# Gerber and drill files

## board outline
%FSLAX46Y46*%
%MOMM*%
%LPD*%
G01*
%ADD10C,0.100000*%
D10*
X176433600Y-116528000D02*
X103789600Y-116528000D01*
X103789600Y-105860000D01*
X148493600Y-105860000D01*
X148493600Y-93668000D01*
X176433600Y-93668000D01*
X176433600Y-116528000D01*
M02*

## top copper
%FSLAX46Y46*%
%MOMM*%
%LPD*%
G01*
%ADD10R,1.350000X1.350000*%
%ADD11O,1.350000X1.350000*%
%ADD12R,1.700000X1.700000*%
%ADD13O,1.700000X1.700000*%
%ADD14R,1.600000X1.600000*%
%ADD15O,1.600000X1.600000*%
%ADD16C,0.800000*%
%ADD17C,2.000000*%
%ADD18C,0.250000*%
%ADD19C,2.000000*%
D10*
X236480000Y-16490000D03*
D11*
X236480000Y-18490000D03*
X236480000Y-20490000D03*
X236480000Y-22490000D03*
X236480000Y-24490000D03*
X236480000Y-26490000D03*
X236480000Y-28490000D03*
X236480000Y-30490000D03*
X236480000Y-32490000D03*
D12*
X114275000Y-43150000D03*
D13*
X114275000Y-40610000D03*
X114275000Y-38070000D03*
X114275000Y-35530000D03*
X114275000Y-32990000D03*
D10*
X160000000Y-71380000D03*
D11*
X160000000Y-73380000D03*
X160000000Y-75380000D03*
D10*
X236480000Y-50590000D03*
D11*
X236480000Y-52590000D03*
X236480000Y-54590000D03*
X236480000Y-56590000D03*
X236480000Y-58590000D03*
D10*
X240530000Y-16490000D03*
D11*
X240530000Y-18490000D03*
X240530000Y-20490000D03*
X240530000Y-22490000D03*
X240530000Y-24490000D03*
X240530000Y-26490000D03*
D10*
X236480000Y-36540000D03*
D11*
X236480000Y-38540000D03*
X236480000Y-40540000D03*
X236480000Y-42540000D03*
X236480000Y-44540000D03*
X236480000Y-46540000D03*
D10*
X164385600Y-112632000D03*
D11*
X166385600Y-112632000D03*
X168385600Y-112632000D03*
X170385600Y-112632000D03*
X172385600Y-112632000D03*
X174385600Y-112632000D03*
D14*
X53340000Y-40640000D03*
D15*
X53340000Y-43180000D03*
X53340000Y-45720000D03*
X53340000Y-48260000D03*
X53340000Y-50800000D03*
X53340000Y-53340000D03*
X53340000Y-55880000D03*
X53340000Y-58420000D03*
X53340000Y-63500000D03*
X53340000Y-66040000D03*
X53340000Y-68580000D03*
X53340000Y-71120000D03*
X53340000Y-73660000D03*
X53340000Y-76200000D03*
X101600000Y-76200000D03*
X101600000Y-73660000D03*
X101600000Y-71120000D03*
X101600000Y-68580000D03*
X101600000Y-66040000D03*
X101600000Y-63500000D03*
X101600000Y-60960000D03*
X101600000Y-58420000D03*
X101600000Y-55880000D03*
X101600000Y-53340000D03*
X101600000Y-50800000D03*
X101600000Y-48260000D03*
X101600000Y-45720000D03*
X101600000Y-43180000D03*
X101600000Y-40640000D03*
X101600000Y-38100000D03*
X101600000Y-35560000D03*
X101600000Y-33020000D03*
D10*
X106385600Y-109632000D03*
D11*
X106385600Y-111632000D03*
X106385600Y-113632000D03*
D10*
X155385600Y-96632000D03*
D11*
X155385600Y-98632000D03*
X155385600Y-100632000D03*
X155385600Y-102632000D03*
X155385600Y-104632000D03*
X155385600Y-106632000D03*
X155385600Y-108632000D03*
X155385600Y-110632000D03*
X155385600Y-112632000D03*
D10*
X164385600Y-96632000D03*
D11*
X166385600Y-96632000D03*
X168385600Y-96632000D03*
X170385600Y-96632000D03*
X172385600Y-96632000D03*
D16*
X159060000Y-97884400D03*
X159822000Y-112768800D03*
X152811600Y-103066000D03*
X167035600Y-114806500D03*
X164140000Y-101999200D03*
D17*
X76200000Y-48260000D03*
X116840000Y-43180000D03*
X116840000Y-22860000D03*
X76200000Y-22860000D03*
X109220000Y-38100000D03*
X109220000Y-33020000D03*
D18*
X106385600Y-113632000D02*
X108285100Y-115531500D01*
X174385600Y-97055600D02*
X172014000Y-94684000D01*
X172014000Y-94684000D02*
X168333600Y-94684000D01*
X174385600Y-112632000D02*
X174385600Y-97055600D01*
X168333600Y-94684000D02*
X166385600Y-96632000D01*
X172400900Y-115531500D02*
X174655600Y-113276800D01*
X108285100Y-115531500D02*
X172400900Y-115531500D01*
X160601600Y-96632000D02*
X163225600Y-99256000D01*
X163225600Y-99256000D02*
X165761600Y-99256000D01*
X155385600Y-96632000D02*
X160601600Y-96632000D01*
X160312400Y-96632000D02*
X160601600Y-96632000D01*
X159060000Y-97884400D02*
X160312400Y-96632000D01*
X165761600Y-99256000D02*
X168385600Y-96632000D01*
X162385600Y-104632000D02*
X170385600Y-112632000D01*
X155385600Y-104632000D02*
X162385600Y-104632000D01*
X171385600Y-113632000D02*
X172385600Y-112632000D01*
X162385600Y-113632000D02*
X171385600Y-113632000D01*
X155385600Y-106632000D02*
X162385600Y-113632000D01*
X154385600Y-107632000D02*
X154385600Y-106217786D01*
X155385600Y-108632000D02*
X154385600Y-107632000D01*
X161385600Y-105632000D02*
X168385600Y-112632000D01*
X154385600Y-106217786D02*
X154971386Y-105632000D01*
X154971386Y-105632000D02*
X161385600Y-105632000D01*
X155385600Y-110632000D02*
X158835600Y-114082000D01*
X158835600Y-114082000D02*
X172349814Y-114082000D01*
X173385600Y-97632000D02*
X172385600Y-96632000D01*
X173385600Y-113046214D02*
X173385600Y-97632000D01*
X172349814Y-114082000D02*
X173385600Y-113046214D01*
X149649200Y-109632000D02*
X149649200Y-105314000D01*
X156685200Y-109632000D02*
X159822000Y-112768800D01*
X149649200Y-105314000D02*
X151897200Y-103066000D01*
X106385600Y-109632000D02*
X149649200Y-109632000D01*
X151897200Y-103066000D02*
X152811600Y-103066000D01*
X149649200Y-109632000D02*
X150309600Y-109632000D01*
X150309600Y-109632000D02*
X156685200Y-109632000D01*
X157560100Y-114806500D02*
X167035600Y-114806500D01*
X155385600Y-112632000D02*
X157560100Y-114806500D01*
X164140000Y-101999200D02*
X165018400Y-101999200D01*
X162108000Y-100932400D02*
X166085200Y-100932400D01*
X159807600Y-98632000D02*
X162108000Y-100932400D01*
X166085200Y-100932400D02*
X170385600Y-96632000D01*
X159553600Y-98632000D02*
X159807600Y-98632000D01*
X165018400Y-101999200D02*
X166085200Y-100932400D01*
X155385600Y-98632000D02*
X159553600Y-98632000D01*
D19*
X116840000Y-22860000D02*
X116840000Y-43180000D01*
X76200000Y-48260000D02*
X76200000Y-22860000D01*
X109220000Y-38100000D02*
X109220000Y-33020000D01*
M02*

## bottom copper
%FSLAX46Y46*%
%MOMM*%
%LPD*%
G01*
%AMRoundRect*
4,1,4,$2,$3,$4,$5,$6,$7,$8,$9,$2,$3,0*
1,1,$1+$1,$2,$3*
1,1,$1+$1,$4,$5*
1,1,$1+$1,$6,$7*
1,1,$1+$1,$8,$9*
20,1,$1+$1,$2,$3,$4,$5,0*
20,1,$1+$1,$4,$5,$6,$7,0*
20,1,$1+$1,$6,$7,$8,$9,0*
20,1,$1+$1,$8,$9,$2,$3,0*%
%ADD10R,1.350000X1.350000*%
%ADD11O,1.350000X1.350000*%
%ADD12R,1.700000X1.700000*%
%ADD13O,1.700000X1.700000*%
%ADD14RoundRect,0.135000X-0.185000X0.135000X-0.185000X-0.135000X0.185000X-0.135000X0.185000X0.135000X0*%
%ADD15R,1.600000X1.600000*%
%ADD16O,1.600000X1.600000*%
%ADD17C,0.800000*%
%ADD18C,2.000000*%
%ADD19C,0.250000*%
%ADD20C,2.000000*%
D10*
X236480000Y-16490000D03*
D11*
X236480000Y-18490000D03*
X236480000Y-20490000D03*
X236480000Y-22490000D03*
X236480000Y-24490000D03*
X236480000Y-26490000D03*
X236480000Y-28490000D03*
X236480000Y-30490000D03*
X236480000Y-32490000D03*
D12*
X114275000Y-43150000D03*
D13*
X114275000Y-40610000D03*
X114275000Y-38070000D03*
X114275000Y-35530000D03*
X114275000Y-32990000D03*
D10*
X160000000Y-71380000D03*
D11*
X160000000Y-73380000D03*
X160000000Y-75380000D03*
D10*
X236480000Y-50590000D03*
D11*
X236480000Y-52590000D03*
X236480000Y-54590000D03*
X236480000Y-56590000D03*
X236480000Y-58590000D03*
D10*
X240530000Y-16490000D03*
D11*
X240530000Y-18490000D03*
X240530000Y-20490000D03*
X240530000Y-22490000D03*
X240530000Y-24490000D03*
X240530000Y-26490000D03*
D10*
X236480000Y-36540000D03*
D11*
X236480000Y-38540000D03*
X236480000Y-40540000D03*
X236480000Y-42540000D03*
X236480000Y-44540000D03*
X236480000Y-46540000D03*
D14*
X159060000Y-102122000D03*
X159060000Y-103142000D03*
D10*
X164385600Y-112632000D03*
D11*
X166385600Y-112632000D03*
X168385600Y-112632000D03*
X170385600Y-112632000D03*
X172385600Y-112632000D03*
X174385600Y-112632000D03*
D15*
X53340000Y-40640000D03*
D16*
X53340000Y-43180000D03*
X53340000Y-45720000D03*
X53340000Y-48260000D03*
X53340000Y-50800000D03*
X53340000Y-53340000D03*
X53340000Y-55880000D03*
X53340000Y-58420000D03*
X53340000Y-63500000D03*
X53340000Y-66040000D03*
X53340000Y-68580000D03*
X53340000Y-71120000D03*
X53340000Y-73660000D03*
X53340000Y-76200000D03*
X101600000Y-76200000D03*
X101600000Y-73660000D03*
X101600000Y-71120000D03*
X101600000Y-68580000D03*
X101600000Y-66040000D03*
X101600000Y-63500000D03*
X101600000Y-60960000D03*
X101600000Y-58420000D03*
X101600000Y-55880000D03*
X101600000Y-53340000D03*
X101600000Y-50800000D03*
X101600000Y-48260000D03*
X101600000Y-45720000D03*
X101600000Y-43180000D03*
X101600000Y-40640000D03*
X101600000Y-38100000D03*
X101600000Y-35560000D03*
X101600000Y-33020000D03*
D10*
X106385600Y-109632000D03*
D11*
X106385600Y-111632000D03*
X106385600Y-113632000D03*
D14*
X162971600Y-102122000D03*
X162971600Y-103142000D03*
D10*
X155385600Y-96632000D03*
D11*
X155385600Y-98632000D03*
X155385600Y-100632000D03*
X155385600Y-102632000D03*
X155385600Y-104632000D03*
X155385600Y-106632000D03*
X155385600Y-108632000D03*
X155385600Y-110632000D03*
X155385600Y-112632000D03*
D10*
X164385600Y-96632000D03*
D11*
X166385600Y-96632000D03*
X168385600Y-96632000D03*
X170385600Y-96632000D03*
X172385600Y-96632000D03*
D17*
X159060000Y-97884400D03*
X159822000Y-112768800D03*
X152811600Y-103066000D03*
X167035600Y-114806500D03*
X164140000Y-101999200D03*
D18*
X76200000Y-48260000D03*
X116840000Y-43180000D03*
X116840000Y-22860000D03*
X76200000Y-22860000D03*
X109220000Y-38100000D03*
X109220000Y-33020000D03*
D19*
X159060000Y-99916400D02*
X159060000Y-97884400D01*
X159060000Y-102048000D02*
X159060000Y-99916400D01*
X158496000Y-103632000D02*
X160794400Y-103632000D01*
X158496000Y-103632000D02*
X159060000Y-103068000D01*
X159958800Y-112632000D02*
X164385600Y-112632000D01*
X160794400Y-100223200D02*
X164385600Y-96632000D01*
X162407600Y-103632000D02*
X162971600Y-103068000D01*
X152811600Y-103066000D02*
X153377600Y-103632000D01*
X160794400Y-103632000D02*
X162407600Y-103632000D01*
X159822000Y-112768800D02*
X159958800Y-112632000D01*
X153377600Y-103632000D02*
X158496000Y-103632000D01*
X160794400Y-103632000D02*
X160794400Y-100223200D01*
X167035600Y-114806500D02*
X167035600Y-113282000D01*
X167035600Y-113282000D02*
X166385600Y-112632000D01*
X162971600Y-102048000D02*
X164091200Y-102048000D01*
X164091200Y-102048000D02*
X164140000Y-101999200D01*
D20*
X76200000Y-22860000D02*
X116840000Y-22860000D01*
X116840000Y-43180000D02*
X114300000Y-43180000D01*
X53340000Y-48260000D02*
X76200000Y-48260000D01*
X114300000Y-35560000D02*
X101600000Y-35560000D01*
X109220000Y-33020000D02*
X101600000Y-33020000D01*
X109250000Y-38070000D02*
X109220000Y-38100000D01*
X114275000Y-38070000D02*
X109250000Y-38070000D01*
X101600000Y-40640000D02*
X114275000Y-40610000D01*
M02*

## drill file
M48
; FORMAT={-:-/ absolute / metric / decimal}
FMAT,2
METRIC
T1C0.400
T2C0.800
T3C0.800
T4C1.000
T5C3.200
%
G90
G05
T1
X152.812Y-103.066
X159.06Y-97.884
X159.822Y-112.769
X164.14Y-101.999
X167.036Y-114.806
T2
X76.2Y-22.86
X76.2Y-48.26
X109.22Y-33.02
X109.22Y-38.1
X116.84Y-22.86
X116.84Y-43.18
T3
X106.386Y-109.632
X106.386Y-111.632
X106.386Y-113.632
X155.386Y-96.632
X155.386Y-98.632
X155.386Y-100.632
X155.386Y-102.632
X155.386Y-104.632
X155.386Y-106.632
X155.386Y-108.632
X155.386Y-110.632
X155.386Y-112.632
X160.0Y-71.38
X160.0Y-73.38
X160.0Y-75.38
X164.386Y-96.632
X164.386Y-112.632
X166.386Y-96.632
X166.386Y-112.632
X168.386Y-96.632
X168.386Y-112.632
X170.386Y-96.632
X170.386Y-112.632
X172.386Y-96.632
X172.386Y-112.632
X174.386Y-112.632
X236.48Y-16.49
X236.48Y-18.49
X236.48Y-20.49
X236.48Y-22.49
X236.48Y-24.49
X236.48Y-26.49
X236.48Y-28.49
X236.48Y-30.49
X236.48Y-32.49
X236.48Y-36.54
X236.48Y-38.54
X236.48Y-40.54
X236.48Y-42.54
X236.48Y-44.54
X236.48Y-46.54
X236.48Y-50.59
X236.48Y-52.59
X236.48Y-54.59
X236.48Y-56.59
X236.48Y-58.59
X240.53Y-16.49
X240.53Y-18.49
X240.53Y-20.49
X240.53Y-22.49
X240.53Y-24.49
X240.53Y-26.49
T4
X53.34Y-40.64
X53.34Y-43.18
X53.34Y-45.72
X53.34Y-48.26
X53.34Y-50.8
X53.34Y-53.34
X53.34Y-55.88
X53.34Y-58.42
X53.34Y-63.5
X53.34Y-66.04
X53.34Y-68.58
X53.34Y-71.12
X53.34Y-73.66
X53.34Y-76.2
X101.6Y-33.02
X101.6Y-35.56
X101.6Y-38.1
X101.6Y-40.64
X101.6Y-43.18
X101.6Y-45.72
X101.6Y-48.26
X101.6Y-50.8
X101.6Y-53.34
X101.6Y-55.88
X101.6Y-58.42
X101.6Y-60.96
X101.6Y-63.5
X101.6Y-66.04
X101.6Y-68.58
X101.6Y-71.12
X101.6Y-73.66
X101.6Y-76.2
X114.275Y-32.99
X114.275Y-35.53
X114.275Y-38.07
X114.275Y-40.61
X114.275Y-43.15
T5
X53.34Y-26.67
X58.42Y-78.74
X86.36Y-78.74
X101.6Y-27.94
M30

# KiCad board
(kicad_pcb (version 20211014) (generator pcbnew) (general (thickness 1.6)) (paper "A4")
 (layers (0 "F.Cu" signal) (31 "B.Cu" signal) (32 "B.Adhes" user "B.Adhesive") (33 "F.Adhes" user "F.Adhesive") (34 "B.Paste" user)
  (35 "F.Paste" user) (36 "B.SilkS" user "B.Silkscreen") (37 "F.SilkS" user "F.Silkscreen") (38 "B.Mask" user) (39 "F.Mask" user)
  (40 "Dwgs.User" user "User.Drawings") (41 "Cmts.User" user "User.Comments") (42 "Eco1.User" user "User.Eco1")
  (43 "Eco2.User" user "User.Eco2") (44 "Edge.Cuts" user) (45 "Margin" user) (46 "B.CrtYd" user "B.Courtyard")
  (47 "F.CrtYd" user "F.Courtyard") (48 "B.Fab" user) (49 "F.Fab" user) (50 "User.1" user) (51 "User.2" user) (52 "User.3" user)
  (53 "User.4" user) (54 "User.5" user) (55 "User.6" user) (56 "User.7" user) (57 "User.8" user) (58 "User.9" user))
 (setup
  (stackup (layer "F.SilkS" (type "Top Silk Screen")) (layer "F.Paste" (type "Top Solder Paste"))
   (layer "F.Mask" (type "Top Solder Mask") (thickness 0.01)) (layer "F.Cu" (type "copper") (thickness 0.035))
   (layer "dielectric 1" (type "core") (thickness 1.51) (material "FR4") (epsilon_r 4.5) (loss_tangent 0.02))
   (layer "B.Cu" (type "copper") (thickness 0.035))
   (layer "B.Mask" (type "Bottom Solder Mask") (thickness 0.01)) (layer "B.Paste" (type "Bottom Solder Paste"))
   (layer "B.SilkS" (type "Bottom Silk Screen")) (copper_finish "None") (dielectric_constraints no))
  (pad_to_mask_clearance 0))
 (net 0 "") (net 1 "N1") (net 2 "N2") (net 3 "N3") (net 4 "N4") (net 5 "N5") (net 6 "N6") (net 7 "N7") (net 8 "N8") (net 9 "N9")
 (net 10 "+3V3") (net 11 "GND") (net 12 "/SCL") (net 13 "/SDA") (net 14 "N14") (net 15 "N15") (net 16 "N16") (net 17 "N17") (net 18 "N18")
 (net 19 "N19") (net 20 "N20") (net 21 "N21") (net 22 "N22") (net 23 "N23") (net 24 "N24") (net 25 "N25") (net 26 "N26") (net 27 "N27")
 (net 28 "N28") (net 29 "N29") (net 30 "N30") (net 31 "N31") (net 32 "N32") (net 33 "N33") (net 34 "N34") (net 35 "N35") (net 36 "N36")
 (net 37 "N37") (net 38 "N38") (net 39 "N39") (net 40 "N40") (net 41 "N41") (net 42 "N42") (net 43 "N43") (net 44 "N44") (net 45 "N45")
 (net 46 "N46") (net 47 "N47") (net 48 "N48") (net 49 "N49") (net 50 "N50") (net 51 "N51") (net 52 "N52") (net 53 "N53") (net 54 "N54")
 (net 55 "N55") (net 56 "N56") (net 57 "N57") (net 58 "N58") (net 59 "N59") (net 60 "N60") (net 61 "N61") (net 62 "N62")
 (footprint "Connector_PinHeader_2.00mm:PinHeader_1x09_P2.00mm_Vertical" (layer "F.Cu") (at 236.48 16.49)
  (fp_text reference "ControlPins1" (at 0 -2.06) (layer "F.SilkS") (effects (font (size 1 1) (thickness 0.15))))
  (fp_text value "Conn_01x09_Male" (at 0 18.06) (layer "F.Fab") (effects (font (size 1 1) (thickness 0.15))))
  (pad "1" thru_hole rect (at 0 0) (size 1.35 1.35) (drill 0.8) (layers *.Cu *.Mask) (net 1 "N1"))
  (pad "2" thru_hole oval (at 0 2) (size 1.35 1.35) (drill 0.8) (layers *.Cu *.Mask) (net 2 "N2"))
  (pad "3" thru_hole oval (at 0 4) (size 1.35 1.35) (drill 0.8) (layers *.Cu *.Mask) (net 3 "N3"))
  (pad "4" thru_hole oval (at 0 6) (size 1.35 1.35) (drill 0.8) (layers *.Cu *.Mask) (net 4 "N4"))
  (pad "5" thru_hole oval (at 0 8) (size 1.35 1.35) (drill 0.8) (layers *.Cu *.Mask) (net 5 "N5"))
  (pad "6" thru_hole oval (at 0 10) (size 1.35 1.35) (drill 0.8) (layers *.Cu *.Mask) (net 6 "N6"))
  (pad "7" thru_hole oval (at 0 12) (size 1.35 1.35) (drill 0.8) (layers *.Cu *.Mask) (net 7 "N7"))
  (pad "8" thru_hole oval (at 0 14) (size 1.35 1.35) (drill 0.8) (layers *.Cu *.Mask) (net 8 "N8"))
  (pad "9" thru_hole oval (at 0 16) (size 1.35 1.35) (drill 0.8) (layers *.Cu *.Mask) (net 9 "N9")))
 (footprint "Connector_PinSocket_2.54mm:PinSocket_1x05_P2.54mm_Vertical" (layer "F.Cu") (at 114.275 43.15 180)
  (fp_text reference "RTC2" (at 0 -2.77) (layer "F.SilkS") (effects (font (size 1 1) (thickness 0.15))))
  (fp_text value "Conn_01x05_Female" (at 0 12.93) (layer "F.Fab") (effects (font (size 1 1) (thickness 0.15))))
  (pad "1" thru_hole rect (at 0 0 180) (size 1.7 1.7) (drill 1) (layers *.Cu *.Mask) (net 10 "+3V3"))
  (pad "2" thru_hole oval (at 0 2.54 180) (size 1.7 1.7) (drill 1) (layers *.Cu *.Mask) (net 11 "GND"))
  (pad "3" thru_hole oval (at 0 5.08 180) (size 1.7 1.7) (drill 1) (layers *.Cu *.Mask) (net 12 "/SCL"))
  (pad "4" thru_hole oval (at 0 7.62 180) (size 1.7 1.7) (drill 1) (layers *.Cu *.Mask) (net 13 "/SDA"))
  (pad "5" thru_hole oval (at 0 10.16 180) (size 1.7 1.7) (drill 1) (layers *.Cu *.Mask) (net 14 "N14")))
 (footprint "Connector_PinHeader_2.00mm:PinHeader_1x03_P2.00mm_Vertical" (layer "F.Cu") (at 160 71.38)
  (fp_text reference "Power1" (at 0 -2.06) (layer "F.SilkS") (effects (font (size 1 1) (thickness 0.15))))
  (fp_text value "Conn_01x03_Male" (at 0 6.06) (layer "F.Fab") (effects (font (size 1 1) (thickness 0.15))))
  (pad "1" thru_hole rect (at 0 0) (size 1.35 1.35) (drill 0.8) (layers *.Cu *.Mask) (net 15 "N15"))
  (pad "2" thru_hole oval (at 0 2) (size 1.35 1.35) (drill 0.8) (layers *.Cu *.Mask) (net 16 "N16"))
  (pad "3" thru_hole oval (at 0 4) (size 1.35 1.35) (drill 0.8) (layers *.Cu *.Mask) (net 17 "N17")))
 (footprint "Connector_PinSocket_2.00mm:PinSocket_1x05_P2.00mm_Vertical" (layer "F.Cu") (at 236.48 50.59)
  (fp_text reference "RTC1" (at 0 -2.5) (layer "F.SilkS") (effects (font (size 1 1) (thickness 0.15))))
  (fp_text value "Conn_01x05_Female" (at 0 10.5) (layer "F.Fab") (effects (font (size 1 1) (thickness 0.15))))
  (pad "1" thru_hole rect (at 0 0) (size 1.35 1.35) (drill 0.8) (layers *.Cu *.Mask) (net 15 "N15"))
  (pad "2" thru_hole oval (at 0 2) (size 1.35 1.35) (drill 0.8) (layers *.Cu *.Mask) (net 17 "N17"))
  (pad "3" thru_hole oval (at 0 4) (size 1.35 1.35) (drill 0.8) (layers *.Cu *.Mask) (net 1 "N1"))
  (pad "4" thru_hole oval (at 0 6) (size 1.35 1.35) (drill 0.8) (layers *.Cu *.Mask) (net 2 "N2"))
  (pad "5" thru_hole oval (at 0 8) (size 1.35 1.35) (drill 0.8) (layers *.Cu *.Mask) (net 8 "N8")))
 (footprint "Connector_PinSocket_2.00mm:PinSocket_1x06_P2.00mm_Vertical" (layer "F.Cu") (at 240.53 16.49)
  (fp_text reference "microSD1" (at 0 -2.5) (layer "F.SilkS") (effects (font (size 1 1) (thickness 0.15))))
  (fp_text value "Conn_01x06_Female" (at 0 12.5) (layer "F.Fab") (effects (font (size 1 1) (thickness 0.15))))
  (pad "1" thru_hole rect (at 0 0) (size 1.35 1.35) (drill 0.8) (layers *.Cu *.Mask) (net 15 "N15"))
  (pad "2" thru_hole oval (at 0 2) (size 1.35 1.35) (drill 0.8) (layers *.Cu *.Mask) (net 9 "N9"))
  (pad "3" thru_hole oval (at 0 4) (size 1.35 1.35) (drill 0.8) (layers *.Cu *.Mask) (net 7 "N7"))
  (pad "4" thru_hole oval (at 0 6) (size 1.35 1.35) (drill 0.8) (layers *.Cu *.Mask) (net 5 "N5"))
  (pad "5" thru_hole oval (at 0 8) (size 1.35 1.35) (drill 0.8) (layers *.Cu *.Mask) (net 6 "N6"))
  (pad "6" thru_hole oval (at 0 10) (size 1.35 1.35) (drill 0.8) (layers *.Cu *.Mask) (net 17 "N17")))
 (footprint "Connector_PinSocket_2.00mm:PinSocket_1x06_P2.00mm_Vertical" (layer "F.Cu") (at 236.48 36.54)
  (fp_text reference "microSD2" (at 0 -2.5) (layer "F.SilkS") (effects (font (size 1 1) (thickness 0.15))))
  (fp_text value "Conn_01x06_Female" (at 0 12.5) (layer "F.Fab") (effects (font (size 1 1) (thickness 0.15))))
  (pad "1" thru_hole rect (at 0 0) (size 1.35 1.35) (drill 0.8) (layers *.Cu *.Mask) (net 10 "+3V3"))
  (pad "2" thru_hole oval (at 0 2) (size 1.35 1.35) (drill 0.8) (layers *.Cu *.Mask) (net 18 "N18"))
  (pad "3" thru_hole oval (at 0 4) (size 1.35 1.35) (drill 0.8) (layers *.Cu *.Mask) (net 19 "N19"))
  (pad "4" thru_hole oval (at 0 6) (size 1.35 1.35) (drill 0.8) (layers *.Cu *.Mask) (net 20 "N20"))
  (pad "5" thru_hole oval (at 0 8) (size 1.35 1.35) (drill 0.8) (layers *.Cu *.Mask) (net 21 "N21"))
  (pad "6" thru_hole oval (at 0 10) (size 1.35 1.35) (drill 0.8) (layers *.Cu *.Mask) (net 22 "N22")))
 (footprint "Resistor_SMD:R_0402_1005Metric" (layer "B.Cu") (at 159.06 102.632 -90)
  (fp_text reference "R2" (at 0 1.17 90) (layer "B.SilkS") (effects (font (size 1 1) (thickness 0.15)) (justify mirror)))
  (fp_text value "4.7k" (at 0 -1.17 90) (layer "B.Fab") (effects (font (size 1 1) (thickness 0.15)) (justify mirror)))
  (pad "1" smd roundrect (at -0.51 0 270) (size 0.54 0.64) (layers "B.Cu" "B.Paste" "B.Mask") (roundrect_rratio 0.25) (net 1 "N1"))
  (pad "2" smd roundrect (at 0.51 0 270) (size 0.54 0.64) (layers "B.Cu" "B.Paste" "B.Mask") (roundrect_rratio 0.25) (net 15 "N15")))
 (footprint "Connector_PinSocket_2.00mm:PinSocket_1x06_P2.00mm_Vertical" (layer "B.Cu") (at 164.3856 112.632 -90)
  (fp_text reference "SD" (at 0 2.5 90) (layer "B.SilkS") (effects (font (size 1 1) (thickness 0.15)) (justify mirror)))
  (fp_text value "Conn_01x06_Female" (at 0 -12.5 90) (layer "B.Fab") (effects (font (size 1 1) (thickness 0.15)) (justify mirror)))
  (pad "1" thru_hole rect (at 0 0 270) (size 1.35 1.35) (drill 0.8) (layers *.Cu *.Mask) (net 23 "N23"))
  (pad "2" thru_hole oval (at 0 -2 270) (size 1.35 1.35) (drill 0.8) (layers *.Cu *.Mask) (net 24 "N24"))
  (pad "3" thru_hole oval (at 0 -4 270) (size 1.35 1.35) (drill 0.8) (layers *.Cu *.Mask) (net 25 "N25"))
  (pad "4" thru_hole oval (at 0 -6 270) (size 1.35 1.35) (drill 0.8) (layers *.Cu *.Mask) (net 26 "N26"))
  (pad "5" thru_hole oval (at 0 -8 270) (size 1.35 1.35) (drill 0.8) (layers *.Cu *.Mask) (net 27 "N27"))
  (pad "6" thru_hole oval (at 0 -10 270) (size 1.35 1.35) (drill 0.8) (layers *.Cu *.Mask) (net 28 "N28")))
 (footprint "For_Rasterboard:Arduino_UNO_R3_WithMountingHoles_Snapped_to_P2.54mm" (layer "B.Cu") (at 53.34 40.64 -90)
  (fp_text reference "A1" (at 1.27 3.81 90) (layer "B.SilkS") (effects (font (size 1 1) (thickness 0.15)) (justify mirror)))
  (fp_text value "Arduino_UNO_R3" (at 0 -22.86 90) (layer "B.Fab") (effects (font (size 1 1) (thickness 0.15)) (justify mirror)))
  (pad "" np_thru_hole circle (at 38.1 -5.08 180) (size 3.2 3.2) (drill 3.2) (layers *.Cu *.Mask))
  (pad "" np_thru_hole circle (at -13.97 0 180) (size 3.2 3.2) (drill 3.2) (layers *.Cu *.Mask))
  (pad "" np_thru_hole circle (at 38.1 -33.02 180) (size 3.2 3.2) (drill 3.2) (layers *.Cu *.Mask))
  (pad "" np_thru_hole circle (at -12.7 -48.26 180) (size 3.2 3.2) (drill 3.2) (layers *.Cu *.Mask))
  (pad "1" thru_hole rect (at 0 0 180) (size 1.6 1.6) (drill 1) (layers *.Cu *.Mask) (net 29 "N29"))
  (pad "2" thru_hole oval (at 2.54 0 180) (size 1.6 1.6) (drill 1) (layers *.Cu *.Mask) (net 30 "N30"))
  (pad "3" thru_hole oval (at 5.08 0 180) (size 1.6 1.6) (drill 1) (layers *.Cu *.Mask) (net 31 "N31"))
  (pad "4" thru_hole oval (at 7.62 0 180) (size 1.6 1.6) (drill 1) (layers *.Cu *.Mask) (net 10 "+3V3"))
  (pad "5" thru_hole oval (at 10.16 0 180) (size 1.6 1.6) (drill 1) (layers *.Cu *.Mask) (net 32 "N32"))
  (pad "6" thru_hole oval (at 12.7 0 180) (size 1.6 1.6) (drill 1) (layers *.Cu *.Mask) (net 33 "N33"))
  (pad "7" thru_hole oval (at 15.24 0 180) (size 1.6 1.6) (drill 1) (layers *.Cu *.Mask) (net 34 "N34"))
  (pad "8" thru_hole oval (at 17.78 0 180) (size 1.6 1.6) (drill 1) (layers *.Cu *.Mask) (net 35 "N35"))
  (pad "9" thru_hole oval (at 22.86 0 180) (size 1.6 1.6) (drill 1) (layers *.Cu *.Mask) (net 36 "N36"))
  (pad "10" thru_hole oval (at 25.4 0 180) (size 1.6 1.6) (drill 1) (layers *.Cu *.Mask) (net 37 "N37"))
  (pad "11" thru_hole oval (at 27.94 0 180) (size 1.6 1.6) (drill 1) (layers *.Cu *.Mask) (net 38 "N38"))
  (pad "12" thru_hole oval (at 30.48 0 180) (size 1.6 1.6) (drill 1) (layers *.Cu *.Mask) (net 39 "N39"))
  (pad "13" thru_hole oval (at 33.02 0 180) (size 1.6 1.6) (drill 1) (layers *.Cu *.Mask) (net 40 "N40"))
  (pad "14" thru_hole oval (at 35.56 0 180) (size 1.6 1.6) (drill 1) (layers *.Cu *.Mask) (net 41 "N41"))
  (pad "15" thru_hole oval (at 35.56 -48.26 180) (size 1.6 1.6) (drill 1) (layers *.Cu *.Mask) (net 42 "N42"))
  (pad "16" thru_hole oval (at 33.02 -48.26 180) (size 1.6 1.6) (drill 1) (layers *.Cu *.Mask) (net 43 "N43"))
  (pad "17" thru_hole oval (at 30.48 -48.26 180) (size 1.6 1.6) (drill 1) (layers *.Cu *.Mask) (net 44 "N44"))
  (pad "18" thru_hole oval (at 27.94 -48.26 180) (size 1.6 1.6) (drill 1) (layers *.Cu *.Mask) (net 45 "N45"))
  (pad "19" thru_hole oval (at 25.4 -48.26 180) (size 1.6 1.6) (drill 1) (layers *.Cu *.Mask) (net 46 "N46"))
  (pad "20" thru_hole oval (at 22.86 -48.26 180) (size 1.6 1.6) (drill 1) (layers *.Cu *.Mask) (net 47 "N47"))
  (pad "21" thru_hole oval (at 20.32 -48.26 180) (size 1.6 1.6) (drill 1) (layers *.Cu *.Mask) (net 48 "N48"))
  (pad "22" thru_hole oval (at 17.78 -48.26 180) (size 1.6 1.6) (drill 1) (layers *.Cu *.Mask) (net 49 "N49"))
  (pad "23" thru_hole oval (at 15.24 -48.26 180) (size 1.6 1.6) (drill 1) (layers *.Cu *.Mask) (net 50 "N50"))
  (pad "24" thru_hole oval (at 12.7 -48.26 180) (size 1.6 1.6) (drill 1) (layers *.Cu *.Mask) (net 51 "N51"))
  (pad "25" thru_hole oval (at 10.16 -48.26 180) (size 1.6 1.6) (drill 1) (layers *.Cu *.Mask) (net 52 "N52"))
  (pad "26" thru_hole oval (at 7.62 -48.26 180) (size 1.6 1.6) (drill 1) (layers *.Cu *.Mask) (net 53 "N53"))
  (pad "27" thru_hole oval (at 5.08 -48.26 180) (size 1.6 1.6) (drill 1) (layers *.Cu *.Mask) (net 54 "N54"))
  (pad "28" thru_hole oval (at 2.54 -48.26 180) (size 1.6 1.6) (drill 1) (layers *.Cu *.Mask) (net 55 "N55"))
  (pad "29" thru_hole oval (at 0 -48.26 180) (size 1.6 1.6) (drill 1) (layers *.Cu *.Mask) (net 11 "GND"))
  (pad "30" thru_hole oval (at -2.54 -48.26 180) (size 1.6 1.6) (drill 1) (layers *.Cu *.Mask) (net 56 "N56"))
  (pad "31" thru_hole oval (at -5.08 -48.26 180) (size 1.6 1.6) (drill 1) (layers *.Cu *.Mask) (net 13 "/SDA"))
  (pad "32" thru_hole oval (at -7.62 -48.26 180) (size 1.6 1.6) (drill 1) (layers *.Cu *.Mask) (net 12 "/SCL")))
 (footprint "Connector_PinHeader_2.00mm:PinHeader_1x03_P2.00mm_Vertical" (layer "B.Cu") (at 106.3856 109.632 180)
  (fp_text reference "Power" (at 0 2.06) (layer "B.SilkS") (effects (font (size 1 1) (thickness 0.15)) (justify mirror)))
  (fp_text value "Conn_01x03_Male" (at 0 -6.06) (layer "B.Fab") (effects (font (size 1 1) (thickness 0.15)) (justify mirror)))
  (pad "1" thru_hole rect (at 0 0 180) (size 1.35 1.35) (drill 0.8) (layers *.Cu *.Mask) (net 23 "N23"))
  (pad "2" thru_hole oval (at 0 -2 180) (size 1.35 1.35) (drill 0.8) (layers *.Cu *.Mask) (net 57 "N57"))
  (pad "3" thru_hole oval (at 0 -4 180) (size 1.35 1.35) (drill 0.8) (layers *.Cu *.Mask) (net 28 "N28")))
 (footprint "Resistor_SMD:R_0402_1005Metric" (layer "B.Cu") (at 162.9716 102.632 -90)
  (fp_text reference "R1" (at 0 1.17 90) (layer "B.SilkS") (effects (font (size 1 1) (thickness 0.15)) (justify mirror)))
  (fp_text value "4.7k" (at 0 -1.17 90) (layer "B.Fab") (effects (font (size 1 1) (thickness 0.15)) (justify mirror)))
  (pad "1" smd roundrect (at -0.51 0 270) (size 0.54 0.64) (layers "B.Cu" "B.Paste" "B.Mask") (roundrect_rratio 0.25) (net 2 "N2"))
  (pad "2" smd roundrect (at 0.51 0 270) (size 0.54 0.64) (layers "B.Cu" "B.Paste" "B.Mask") (roundrect_rratio 0.25) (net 15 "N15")))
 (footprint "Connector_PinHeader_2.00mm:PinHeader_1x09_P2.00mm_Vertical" (layer "B.Cu") (at 155.3856 96.632 180)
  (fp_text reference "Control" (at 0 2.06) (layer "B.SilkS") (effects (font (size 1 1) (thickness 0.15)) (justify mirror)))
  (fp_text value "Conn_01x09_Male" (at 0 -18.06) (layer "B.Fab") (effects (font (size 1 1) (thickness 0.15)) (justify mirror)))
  (pad "1" thru_hole rect (at 0 0 180) (size 1.35 1.35) (drill 0.8) (layers *.Cu *.Mask) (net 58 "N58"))
  (pad "2" thru_hole oval (at 0 -2 180) (size 1.35 1.35) (drill 0.8) (layers *.Cu *.Mask) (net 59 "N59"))
  (pad "3" thru_hole oval (at 0 -4 180) (size 1.35 1.35) (drill 0.8) (layers *.Cu *.Mask) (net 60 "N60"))
  (pad "4" thru_hole oval (at 0 -6 180) (size 1.35 1.35) (drill 0.8) (layers *.Cu *.Mask) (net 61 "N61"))
  (pad "5" thru_hole oval (at 0 -8 180) (size 1.35 1.35) (drill 0.8) (layers *.Cu *.Mask) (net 26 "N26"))
  (pad "6" thru_hole oval (at 0 -10 180) (size 1.35 1.35) (drill 0.8) (layers *.Cu *.Mask) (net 27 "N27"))
  (pad "7" thru_hole oval (at 0 -12 180) (size 1.35 1.35) (drill 0.8) (layers *.Cu *.Mask) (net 25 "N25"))
  (pad "8" thru_hole oval (at 0 -14 180) (size 1.35 1.35) (drill 0.8) (layers *.Cu *.Mask) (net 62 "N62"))
  (pad "9" thru_hole oval (at 0 -16 180) (size 1.35 1.35) (drill 0.8) (layers *.Cu *.Mask) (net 24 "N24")))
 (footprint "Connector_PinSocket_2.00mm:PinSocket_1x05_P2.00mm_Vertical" (layer "B.Cu") (at 164.3856 96.632 -90)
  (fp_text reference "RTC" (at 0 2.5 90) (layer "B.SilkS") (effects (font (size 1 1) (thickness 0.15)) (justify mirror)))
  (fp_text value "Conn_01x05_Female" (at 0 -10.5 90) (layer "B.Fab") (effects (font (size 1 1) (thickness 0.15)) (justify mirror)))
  (pad "1" thru_hole rect (at 0 0 270) (size 1.35 1.35) (drill 0.8) (layers *.Cu *.Mask) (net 23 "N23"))
  (pad "2" thru_hole oval (at 0 -2 270) (size 1.35 1.35) (drill 0.8) (layers *.Cu *.Mask) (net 28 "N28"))
  (pad "3" thru_hole oval (at 0 -4 270) (size 1.35 1.35) (drill 0.8) (layers *.Cu *.Mask) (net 58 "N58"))
  (pad "4" thru_hole oval (at 0 -6 270) (size 1.35 1.35) (drill 0.8) (layers *.Cu *.Mask) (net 59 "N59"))
  (pad "5" thru_hole oval (at 0 -8 270) (size 1.35 1.35) (drill 0.8) (layers *.Cu *.Mask) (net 62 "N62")))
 (gr_poly
  (pts (xy 176.4336 116.528) (xy 103.7896 116.528) (xy 103.7896 105.86) (xy 148.4936 105.86) (xy 148.4936 93.668) (xy 176.4336 93.668))
  (layer "Edge.Cuts") (width 0.1) (fill none))
 (segment (start 106.3856 113.632) (end 108.2851 115.5315) (width 0.25) (layer "F.Cu") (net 28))
 (segment (start 174.3856 97.0556) (end 172.014 94.684) (width 0.25) (layer "F.Cu") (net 28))
 (segment (start 172.014 94.684) (end 168.3336 94.684) (width 0.25) (layer "F.Cu") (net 28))
 (segment (start 174.3856 112.632) (end 174.3856 97.0556) (width 0.25) (layer "F.Cu") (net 28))
 (segment (start 168.3336 94.684) (end 166.3856 96.632) (width 0.25) (layer "F.Cu") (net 28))
 (segment (start 172.4009 115.5315) (end 174.6556 113.2768) (width 0.25) (layer "F.Cu") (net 28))
 (segment (start 108.2851 115.5315) (end 172.4009 115.5315) (width 0.25) (layer "F.Cu") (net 28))
 (segment (start 160.6016 96.632) (end 163.2256 99.256) (width 0.25) (layer "F.Cu") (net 58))
 (segment (start 163.2256 99.256) (end 165.7616 99.256) (width 0.25) (layer "F.Cu") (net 58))
 (segment (start 155.3856 96.632) (end 160.6016 96.632) (width 0.25) (layer "F.Cu") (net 58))
 (segment (start 160.3124 96.632) (end 160.6016 96.632) (width 0.25) (layer "F.Cu") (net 58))
 (segment (start 159.06 97.8844) (end 160.3124 96.632) (width 0.25) (layer "F.Cu") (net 58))
 (segment (start 165.7616 99.256) (end 168.3856 96.632) (width 0.25) (layer "F.Cu") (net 58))
 (via (at 159.06 97.8844) (size 0.8) (drill 0.4) (layers "F.Cu" "B.Cu") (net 58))
 (segment (start 159.06 99.9164) (end 159.06 97.8844) (width 0.25) (layer "B.Cu") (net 58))
 (segment (start 159.06 102.048) (end 159.06 99.9164) (width 0.25) (layer "B.Cu") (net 58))
 (segment (start 162.3856 104.632) (end 170.3856 112.632) (width 0.25) (layer "F.Cu") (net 26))
 (segment (start 155.3856 104.632) (end 162.3856 104.632) (width 0.25) (layer "F.Cu") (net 26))
 (segment (start 171.3856 113.632) (end 172.3856 112.632) (width 0.25) (layer "F.Cu") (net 27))
 (segment (start 162.3856 113.632) (end 171.3856 113.632) (width 0.25) (layer "F.Cu") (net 27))
 (segment (start 155.3856 106.632) (end 162.3856 113.632) (width 0.25) (layer "F.Cu") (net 27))
 (segment (start 154.3856 107.632) (end 154.3856 106.217786) (width 0.25) (layer "F.Cu") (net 25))
 (segment (start 155.3856 108.632) (end 154.3856 107.632) (width 0.25) (layer "F.Cu") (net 25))
 (segment (start 161.3856 105.632) (end 168.3856 112.632) (width 0.25) (layer "F.Cu") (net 25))
 (segment (start 154.3856 106.217786) (end 154.971386 105.632) (width 0.25) (layer "F.Cu") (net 25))
 (segment (start 154.971386 105.632) (end 161.3856 105.632) (width 0.25) (layer "F.Cu") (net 25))
 (segment (start 155.3856 110.632) (end 158.8356 114.082) (width 0.25) (layer "F.Cu") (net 62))
 (segment (start 158.8356 114.082) (end 172.349814 114.082) (width 0.25) (layer "F.Cu") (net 62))
 (segment (start 173.3856 97.632) (end 172.3856 96.632) (width 0.25) (layer "F.Cu") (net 62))
 (segment (start 173.3856 113.046214) (end 173.3856 97.632) (width 0.25) (layer "F.Cu") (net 62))
 (segment (start 172.349814 114.082) (end 173.3856 113.046214) (width 0.25) (layer "F.Cu") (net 62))
 (segment (start 149.6492 109.632) (end 149.6492 105.314) (width 0.25) (layer "F.Cu") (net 23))
 (segment (start 156.6852 109.632) (end 159.822 112.7688) (width 0.25) (layer "F.Cu") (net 23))
 (segment (start 149.6492 105.314) (end 151.8972 103.066) (width 0.25) (layer "F.Cu") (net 23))
 (segment (start 106.3856 109.632) (end 149.6492 109.632) (width 0.25) (layer "F.Cu") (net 23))
 (segment (start 151.8972 103.066) (end 152.8116 103.066) (width 0.25) (layer "F.Cu") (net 23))
 (segment (start 149.6492 109.632) (end 150.3096 109.632) (width 0.25) (layer "F.Cu") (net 23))
 (segment (start 150.3096 109.632) (end 156.6852 109.632) (width 0.25) (layer "F.Cu") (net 23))
 (via (at 159.822 112.7688) (size 0.8) (drill 0.4) (layers "F.Cu" "B.Cu") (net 23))
 (via (at 152.8116 103.066) (size 0.8) (drill 0.4) (layers "F.Cu" "B.Cu") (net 23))
 (segment (start 158.496 103.632) (end 160.7944 103.632) (width 0.25) (layer "B.Cu") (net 23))
 (segment (start 158.496 103.632) (end 159.06 103.068) (width 0.25) (layer "B.Cu") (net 23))
 (segment (start 159.9588 112.632) (end 164.3856 112.632) (width 0.25) (layer "B.Cu") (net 23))
 (segment (start 160.7944 100.2232) (end 164.3856 96.632) (width 0.25) (layer "B.Cu") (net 23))
 (segment (start 162.4076 103.632) (end 162.9716 103.068) (width 0.25) (layer "B.Cu") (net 23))
 (segment (start 152.8116 103.066) (end 153.3776 103.632) (width 0.25) (layer "B.Cu") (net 23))
 (segment (start 160.7944 103.632) (end 162.4076 103.632) (width 0.25) (layer "B.Cu") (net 23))
 (segment (start 159.822 112.7688) (end 159.9588 112.632) (width 0.25) (layer "B.Cu") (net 23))
 (segment (start 153.3776 103.632) (end 158.496 103.632) (width 0.25) (layer "B.Cu") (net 23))
 (segment (start 160.7944 103.632) (end 160.7944 100.2232) (width 0.25) (layer "B.Cu") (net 23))
 (segment (start 157.5601 114.8065) (end 167.0356 114.8065) (width 0.25) (layer "F.Cu") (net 24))
 (segment (start 155.3856 112.632) (end 157.5601 114.8065) (width 0.25) (layer "F.Cu") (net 24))
 (via (at 167.0356 114.8065) (size 0.8) (drill 0.4) (layers "F.Cu" "B.Cu") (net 24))
 (segment (start 167.0356 114.8065) (end 167.0356 113.282) (width 0.25) (layer "B.Cu") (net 24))
 (segment (start 167.0356 113.282) (end 166.3856 112.632) (width 0.25) (layer "B.Cu") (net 24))
 (segment (start 164.14 101.9992) (end 165.0184 101.9992) (width 0.25) (layer "F.Cu") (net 59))
 (segment (start 162.108 100.9324) (end 166.0852 100.9324) (width 0.25) (layer "F.Cu") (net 59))
 (segment (start 159.8076 98.632) (end 162.108 100.9324) (width 0.25) (layer "F.Cu") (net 59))
 (segment (start 166.0852 100.9324) (end 170.3856 96.632) (width 0.25) (layer "F.Cu") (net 59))
 (segment (start 159.5536 98.632) (end 159.8076 98.632) (width 0.25) (layer "F.Cu") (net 59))
 (segment (start 165.0184 101.9992) (end 166.0852 100.9324) (width 0.25) (layer "F.Cu") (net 59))
 (segment (start 155.3856 98.632) (end 159.5536 98.632) (width 0.25) (layer "F.Cu") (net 59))
 (via (at 164.14 101.9992) (size 0.8) (drill 0.4) (layers "F.Cu" "B.Cu") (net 59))
 (segment (start 162.9716 102.048) (end 164.0912 102.048) (width 0.25) (layer "B.Cu") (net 59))
 (segment (start 164.0912 102.048) (end 164.14 101.9992) (width 0.25) (layer "B.Cu") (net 59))
 (segment (start 116.84 22.86) (end 116.84 43.18) (width 2) (layer "F.Cu") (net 10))
 (segment (start 76.2 48.26) (end 76.2 22.86) (width 2) (layer "F.Cu") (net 10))
 (via (at 76.2 48.26) (size 2) (drill 0.8) (layers "F.Cu" "B.Cu") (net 10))
 (via (at 116.84 43.18) (size 2) (drill 0.8) (layers "F.Cu" "B.Cu") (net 10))
 (via (at 116.84 22.86) (size 2) (drill 0.8) (layers "F.Cu" "B.Cu") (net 10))
 (via (at 76.2 22.86) (size 2) (drill 0.8) (layers "F.Cu" "B.Cu") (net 10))
 (segment (start 76.2 22.86) (end 116.84 22.86) (width 2) (layer "B.Cu") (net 10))
 (segment (start 116.84 43.18) (end 114.3 43.18) (width 2) (layer "B.Cu") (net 10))
 (segment (start 53.34 48.26) (end 76.2 48.26) (width 2) (layer "B.Cu") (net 10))
 (segment (start 114.3 35.56) (end 101.6 35.56) (width 2) (layer "B.Cu") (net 13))
 (segment (start 109.22 38.1) (end 109.22 33.02) (width 2) (layer "F.Cu") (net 12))
 (via (at 109.22 38.1) (size 2) (drill 0.8) (layers "F.Cu" "B.Cu") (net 12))
 (via (at 109.22 33.02) (size 2) (drill 0.8) (layers "F.Cu" "B.Cu") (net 12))
 (segment (start 109.22 33.02) (end 101.6 33.02) (width 2) (layer "B.Cu") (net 12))
 (segment (start 109.25 38.07) (end 109.22 38.1) (width 2) (layer "B.Cu") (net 12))
 (segment (start 114.275 38.07) (end 109.25 38.07) (width 2) (layer "B.Cu") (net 12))
 (segment (start 101.6 40.64) (end 114.275 40.61) (width 2) (layer "B.Cu") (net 11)))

